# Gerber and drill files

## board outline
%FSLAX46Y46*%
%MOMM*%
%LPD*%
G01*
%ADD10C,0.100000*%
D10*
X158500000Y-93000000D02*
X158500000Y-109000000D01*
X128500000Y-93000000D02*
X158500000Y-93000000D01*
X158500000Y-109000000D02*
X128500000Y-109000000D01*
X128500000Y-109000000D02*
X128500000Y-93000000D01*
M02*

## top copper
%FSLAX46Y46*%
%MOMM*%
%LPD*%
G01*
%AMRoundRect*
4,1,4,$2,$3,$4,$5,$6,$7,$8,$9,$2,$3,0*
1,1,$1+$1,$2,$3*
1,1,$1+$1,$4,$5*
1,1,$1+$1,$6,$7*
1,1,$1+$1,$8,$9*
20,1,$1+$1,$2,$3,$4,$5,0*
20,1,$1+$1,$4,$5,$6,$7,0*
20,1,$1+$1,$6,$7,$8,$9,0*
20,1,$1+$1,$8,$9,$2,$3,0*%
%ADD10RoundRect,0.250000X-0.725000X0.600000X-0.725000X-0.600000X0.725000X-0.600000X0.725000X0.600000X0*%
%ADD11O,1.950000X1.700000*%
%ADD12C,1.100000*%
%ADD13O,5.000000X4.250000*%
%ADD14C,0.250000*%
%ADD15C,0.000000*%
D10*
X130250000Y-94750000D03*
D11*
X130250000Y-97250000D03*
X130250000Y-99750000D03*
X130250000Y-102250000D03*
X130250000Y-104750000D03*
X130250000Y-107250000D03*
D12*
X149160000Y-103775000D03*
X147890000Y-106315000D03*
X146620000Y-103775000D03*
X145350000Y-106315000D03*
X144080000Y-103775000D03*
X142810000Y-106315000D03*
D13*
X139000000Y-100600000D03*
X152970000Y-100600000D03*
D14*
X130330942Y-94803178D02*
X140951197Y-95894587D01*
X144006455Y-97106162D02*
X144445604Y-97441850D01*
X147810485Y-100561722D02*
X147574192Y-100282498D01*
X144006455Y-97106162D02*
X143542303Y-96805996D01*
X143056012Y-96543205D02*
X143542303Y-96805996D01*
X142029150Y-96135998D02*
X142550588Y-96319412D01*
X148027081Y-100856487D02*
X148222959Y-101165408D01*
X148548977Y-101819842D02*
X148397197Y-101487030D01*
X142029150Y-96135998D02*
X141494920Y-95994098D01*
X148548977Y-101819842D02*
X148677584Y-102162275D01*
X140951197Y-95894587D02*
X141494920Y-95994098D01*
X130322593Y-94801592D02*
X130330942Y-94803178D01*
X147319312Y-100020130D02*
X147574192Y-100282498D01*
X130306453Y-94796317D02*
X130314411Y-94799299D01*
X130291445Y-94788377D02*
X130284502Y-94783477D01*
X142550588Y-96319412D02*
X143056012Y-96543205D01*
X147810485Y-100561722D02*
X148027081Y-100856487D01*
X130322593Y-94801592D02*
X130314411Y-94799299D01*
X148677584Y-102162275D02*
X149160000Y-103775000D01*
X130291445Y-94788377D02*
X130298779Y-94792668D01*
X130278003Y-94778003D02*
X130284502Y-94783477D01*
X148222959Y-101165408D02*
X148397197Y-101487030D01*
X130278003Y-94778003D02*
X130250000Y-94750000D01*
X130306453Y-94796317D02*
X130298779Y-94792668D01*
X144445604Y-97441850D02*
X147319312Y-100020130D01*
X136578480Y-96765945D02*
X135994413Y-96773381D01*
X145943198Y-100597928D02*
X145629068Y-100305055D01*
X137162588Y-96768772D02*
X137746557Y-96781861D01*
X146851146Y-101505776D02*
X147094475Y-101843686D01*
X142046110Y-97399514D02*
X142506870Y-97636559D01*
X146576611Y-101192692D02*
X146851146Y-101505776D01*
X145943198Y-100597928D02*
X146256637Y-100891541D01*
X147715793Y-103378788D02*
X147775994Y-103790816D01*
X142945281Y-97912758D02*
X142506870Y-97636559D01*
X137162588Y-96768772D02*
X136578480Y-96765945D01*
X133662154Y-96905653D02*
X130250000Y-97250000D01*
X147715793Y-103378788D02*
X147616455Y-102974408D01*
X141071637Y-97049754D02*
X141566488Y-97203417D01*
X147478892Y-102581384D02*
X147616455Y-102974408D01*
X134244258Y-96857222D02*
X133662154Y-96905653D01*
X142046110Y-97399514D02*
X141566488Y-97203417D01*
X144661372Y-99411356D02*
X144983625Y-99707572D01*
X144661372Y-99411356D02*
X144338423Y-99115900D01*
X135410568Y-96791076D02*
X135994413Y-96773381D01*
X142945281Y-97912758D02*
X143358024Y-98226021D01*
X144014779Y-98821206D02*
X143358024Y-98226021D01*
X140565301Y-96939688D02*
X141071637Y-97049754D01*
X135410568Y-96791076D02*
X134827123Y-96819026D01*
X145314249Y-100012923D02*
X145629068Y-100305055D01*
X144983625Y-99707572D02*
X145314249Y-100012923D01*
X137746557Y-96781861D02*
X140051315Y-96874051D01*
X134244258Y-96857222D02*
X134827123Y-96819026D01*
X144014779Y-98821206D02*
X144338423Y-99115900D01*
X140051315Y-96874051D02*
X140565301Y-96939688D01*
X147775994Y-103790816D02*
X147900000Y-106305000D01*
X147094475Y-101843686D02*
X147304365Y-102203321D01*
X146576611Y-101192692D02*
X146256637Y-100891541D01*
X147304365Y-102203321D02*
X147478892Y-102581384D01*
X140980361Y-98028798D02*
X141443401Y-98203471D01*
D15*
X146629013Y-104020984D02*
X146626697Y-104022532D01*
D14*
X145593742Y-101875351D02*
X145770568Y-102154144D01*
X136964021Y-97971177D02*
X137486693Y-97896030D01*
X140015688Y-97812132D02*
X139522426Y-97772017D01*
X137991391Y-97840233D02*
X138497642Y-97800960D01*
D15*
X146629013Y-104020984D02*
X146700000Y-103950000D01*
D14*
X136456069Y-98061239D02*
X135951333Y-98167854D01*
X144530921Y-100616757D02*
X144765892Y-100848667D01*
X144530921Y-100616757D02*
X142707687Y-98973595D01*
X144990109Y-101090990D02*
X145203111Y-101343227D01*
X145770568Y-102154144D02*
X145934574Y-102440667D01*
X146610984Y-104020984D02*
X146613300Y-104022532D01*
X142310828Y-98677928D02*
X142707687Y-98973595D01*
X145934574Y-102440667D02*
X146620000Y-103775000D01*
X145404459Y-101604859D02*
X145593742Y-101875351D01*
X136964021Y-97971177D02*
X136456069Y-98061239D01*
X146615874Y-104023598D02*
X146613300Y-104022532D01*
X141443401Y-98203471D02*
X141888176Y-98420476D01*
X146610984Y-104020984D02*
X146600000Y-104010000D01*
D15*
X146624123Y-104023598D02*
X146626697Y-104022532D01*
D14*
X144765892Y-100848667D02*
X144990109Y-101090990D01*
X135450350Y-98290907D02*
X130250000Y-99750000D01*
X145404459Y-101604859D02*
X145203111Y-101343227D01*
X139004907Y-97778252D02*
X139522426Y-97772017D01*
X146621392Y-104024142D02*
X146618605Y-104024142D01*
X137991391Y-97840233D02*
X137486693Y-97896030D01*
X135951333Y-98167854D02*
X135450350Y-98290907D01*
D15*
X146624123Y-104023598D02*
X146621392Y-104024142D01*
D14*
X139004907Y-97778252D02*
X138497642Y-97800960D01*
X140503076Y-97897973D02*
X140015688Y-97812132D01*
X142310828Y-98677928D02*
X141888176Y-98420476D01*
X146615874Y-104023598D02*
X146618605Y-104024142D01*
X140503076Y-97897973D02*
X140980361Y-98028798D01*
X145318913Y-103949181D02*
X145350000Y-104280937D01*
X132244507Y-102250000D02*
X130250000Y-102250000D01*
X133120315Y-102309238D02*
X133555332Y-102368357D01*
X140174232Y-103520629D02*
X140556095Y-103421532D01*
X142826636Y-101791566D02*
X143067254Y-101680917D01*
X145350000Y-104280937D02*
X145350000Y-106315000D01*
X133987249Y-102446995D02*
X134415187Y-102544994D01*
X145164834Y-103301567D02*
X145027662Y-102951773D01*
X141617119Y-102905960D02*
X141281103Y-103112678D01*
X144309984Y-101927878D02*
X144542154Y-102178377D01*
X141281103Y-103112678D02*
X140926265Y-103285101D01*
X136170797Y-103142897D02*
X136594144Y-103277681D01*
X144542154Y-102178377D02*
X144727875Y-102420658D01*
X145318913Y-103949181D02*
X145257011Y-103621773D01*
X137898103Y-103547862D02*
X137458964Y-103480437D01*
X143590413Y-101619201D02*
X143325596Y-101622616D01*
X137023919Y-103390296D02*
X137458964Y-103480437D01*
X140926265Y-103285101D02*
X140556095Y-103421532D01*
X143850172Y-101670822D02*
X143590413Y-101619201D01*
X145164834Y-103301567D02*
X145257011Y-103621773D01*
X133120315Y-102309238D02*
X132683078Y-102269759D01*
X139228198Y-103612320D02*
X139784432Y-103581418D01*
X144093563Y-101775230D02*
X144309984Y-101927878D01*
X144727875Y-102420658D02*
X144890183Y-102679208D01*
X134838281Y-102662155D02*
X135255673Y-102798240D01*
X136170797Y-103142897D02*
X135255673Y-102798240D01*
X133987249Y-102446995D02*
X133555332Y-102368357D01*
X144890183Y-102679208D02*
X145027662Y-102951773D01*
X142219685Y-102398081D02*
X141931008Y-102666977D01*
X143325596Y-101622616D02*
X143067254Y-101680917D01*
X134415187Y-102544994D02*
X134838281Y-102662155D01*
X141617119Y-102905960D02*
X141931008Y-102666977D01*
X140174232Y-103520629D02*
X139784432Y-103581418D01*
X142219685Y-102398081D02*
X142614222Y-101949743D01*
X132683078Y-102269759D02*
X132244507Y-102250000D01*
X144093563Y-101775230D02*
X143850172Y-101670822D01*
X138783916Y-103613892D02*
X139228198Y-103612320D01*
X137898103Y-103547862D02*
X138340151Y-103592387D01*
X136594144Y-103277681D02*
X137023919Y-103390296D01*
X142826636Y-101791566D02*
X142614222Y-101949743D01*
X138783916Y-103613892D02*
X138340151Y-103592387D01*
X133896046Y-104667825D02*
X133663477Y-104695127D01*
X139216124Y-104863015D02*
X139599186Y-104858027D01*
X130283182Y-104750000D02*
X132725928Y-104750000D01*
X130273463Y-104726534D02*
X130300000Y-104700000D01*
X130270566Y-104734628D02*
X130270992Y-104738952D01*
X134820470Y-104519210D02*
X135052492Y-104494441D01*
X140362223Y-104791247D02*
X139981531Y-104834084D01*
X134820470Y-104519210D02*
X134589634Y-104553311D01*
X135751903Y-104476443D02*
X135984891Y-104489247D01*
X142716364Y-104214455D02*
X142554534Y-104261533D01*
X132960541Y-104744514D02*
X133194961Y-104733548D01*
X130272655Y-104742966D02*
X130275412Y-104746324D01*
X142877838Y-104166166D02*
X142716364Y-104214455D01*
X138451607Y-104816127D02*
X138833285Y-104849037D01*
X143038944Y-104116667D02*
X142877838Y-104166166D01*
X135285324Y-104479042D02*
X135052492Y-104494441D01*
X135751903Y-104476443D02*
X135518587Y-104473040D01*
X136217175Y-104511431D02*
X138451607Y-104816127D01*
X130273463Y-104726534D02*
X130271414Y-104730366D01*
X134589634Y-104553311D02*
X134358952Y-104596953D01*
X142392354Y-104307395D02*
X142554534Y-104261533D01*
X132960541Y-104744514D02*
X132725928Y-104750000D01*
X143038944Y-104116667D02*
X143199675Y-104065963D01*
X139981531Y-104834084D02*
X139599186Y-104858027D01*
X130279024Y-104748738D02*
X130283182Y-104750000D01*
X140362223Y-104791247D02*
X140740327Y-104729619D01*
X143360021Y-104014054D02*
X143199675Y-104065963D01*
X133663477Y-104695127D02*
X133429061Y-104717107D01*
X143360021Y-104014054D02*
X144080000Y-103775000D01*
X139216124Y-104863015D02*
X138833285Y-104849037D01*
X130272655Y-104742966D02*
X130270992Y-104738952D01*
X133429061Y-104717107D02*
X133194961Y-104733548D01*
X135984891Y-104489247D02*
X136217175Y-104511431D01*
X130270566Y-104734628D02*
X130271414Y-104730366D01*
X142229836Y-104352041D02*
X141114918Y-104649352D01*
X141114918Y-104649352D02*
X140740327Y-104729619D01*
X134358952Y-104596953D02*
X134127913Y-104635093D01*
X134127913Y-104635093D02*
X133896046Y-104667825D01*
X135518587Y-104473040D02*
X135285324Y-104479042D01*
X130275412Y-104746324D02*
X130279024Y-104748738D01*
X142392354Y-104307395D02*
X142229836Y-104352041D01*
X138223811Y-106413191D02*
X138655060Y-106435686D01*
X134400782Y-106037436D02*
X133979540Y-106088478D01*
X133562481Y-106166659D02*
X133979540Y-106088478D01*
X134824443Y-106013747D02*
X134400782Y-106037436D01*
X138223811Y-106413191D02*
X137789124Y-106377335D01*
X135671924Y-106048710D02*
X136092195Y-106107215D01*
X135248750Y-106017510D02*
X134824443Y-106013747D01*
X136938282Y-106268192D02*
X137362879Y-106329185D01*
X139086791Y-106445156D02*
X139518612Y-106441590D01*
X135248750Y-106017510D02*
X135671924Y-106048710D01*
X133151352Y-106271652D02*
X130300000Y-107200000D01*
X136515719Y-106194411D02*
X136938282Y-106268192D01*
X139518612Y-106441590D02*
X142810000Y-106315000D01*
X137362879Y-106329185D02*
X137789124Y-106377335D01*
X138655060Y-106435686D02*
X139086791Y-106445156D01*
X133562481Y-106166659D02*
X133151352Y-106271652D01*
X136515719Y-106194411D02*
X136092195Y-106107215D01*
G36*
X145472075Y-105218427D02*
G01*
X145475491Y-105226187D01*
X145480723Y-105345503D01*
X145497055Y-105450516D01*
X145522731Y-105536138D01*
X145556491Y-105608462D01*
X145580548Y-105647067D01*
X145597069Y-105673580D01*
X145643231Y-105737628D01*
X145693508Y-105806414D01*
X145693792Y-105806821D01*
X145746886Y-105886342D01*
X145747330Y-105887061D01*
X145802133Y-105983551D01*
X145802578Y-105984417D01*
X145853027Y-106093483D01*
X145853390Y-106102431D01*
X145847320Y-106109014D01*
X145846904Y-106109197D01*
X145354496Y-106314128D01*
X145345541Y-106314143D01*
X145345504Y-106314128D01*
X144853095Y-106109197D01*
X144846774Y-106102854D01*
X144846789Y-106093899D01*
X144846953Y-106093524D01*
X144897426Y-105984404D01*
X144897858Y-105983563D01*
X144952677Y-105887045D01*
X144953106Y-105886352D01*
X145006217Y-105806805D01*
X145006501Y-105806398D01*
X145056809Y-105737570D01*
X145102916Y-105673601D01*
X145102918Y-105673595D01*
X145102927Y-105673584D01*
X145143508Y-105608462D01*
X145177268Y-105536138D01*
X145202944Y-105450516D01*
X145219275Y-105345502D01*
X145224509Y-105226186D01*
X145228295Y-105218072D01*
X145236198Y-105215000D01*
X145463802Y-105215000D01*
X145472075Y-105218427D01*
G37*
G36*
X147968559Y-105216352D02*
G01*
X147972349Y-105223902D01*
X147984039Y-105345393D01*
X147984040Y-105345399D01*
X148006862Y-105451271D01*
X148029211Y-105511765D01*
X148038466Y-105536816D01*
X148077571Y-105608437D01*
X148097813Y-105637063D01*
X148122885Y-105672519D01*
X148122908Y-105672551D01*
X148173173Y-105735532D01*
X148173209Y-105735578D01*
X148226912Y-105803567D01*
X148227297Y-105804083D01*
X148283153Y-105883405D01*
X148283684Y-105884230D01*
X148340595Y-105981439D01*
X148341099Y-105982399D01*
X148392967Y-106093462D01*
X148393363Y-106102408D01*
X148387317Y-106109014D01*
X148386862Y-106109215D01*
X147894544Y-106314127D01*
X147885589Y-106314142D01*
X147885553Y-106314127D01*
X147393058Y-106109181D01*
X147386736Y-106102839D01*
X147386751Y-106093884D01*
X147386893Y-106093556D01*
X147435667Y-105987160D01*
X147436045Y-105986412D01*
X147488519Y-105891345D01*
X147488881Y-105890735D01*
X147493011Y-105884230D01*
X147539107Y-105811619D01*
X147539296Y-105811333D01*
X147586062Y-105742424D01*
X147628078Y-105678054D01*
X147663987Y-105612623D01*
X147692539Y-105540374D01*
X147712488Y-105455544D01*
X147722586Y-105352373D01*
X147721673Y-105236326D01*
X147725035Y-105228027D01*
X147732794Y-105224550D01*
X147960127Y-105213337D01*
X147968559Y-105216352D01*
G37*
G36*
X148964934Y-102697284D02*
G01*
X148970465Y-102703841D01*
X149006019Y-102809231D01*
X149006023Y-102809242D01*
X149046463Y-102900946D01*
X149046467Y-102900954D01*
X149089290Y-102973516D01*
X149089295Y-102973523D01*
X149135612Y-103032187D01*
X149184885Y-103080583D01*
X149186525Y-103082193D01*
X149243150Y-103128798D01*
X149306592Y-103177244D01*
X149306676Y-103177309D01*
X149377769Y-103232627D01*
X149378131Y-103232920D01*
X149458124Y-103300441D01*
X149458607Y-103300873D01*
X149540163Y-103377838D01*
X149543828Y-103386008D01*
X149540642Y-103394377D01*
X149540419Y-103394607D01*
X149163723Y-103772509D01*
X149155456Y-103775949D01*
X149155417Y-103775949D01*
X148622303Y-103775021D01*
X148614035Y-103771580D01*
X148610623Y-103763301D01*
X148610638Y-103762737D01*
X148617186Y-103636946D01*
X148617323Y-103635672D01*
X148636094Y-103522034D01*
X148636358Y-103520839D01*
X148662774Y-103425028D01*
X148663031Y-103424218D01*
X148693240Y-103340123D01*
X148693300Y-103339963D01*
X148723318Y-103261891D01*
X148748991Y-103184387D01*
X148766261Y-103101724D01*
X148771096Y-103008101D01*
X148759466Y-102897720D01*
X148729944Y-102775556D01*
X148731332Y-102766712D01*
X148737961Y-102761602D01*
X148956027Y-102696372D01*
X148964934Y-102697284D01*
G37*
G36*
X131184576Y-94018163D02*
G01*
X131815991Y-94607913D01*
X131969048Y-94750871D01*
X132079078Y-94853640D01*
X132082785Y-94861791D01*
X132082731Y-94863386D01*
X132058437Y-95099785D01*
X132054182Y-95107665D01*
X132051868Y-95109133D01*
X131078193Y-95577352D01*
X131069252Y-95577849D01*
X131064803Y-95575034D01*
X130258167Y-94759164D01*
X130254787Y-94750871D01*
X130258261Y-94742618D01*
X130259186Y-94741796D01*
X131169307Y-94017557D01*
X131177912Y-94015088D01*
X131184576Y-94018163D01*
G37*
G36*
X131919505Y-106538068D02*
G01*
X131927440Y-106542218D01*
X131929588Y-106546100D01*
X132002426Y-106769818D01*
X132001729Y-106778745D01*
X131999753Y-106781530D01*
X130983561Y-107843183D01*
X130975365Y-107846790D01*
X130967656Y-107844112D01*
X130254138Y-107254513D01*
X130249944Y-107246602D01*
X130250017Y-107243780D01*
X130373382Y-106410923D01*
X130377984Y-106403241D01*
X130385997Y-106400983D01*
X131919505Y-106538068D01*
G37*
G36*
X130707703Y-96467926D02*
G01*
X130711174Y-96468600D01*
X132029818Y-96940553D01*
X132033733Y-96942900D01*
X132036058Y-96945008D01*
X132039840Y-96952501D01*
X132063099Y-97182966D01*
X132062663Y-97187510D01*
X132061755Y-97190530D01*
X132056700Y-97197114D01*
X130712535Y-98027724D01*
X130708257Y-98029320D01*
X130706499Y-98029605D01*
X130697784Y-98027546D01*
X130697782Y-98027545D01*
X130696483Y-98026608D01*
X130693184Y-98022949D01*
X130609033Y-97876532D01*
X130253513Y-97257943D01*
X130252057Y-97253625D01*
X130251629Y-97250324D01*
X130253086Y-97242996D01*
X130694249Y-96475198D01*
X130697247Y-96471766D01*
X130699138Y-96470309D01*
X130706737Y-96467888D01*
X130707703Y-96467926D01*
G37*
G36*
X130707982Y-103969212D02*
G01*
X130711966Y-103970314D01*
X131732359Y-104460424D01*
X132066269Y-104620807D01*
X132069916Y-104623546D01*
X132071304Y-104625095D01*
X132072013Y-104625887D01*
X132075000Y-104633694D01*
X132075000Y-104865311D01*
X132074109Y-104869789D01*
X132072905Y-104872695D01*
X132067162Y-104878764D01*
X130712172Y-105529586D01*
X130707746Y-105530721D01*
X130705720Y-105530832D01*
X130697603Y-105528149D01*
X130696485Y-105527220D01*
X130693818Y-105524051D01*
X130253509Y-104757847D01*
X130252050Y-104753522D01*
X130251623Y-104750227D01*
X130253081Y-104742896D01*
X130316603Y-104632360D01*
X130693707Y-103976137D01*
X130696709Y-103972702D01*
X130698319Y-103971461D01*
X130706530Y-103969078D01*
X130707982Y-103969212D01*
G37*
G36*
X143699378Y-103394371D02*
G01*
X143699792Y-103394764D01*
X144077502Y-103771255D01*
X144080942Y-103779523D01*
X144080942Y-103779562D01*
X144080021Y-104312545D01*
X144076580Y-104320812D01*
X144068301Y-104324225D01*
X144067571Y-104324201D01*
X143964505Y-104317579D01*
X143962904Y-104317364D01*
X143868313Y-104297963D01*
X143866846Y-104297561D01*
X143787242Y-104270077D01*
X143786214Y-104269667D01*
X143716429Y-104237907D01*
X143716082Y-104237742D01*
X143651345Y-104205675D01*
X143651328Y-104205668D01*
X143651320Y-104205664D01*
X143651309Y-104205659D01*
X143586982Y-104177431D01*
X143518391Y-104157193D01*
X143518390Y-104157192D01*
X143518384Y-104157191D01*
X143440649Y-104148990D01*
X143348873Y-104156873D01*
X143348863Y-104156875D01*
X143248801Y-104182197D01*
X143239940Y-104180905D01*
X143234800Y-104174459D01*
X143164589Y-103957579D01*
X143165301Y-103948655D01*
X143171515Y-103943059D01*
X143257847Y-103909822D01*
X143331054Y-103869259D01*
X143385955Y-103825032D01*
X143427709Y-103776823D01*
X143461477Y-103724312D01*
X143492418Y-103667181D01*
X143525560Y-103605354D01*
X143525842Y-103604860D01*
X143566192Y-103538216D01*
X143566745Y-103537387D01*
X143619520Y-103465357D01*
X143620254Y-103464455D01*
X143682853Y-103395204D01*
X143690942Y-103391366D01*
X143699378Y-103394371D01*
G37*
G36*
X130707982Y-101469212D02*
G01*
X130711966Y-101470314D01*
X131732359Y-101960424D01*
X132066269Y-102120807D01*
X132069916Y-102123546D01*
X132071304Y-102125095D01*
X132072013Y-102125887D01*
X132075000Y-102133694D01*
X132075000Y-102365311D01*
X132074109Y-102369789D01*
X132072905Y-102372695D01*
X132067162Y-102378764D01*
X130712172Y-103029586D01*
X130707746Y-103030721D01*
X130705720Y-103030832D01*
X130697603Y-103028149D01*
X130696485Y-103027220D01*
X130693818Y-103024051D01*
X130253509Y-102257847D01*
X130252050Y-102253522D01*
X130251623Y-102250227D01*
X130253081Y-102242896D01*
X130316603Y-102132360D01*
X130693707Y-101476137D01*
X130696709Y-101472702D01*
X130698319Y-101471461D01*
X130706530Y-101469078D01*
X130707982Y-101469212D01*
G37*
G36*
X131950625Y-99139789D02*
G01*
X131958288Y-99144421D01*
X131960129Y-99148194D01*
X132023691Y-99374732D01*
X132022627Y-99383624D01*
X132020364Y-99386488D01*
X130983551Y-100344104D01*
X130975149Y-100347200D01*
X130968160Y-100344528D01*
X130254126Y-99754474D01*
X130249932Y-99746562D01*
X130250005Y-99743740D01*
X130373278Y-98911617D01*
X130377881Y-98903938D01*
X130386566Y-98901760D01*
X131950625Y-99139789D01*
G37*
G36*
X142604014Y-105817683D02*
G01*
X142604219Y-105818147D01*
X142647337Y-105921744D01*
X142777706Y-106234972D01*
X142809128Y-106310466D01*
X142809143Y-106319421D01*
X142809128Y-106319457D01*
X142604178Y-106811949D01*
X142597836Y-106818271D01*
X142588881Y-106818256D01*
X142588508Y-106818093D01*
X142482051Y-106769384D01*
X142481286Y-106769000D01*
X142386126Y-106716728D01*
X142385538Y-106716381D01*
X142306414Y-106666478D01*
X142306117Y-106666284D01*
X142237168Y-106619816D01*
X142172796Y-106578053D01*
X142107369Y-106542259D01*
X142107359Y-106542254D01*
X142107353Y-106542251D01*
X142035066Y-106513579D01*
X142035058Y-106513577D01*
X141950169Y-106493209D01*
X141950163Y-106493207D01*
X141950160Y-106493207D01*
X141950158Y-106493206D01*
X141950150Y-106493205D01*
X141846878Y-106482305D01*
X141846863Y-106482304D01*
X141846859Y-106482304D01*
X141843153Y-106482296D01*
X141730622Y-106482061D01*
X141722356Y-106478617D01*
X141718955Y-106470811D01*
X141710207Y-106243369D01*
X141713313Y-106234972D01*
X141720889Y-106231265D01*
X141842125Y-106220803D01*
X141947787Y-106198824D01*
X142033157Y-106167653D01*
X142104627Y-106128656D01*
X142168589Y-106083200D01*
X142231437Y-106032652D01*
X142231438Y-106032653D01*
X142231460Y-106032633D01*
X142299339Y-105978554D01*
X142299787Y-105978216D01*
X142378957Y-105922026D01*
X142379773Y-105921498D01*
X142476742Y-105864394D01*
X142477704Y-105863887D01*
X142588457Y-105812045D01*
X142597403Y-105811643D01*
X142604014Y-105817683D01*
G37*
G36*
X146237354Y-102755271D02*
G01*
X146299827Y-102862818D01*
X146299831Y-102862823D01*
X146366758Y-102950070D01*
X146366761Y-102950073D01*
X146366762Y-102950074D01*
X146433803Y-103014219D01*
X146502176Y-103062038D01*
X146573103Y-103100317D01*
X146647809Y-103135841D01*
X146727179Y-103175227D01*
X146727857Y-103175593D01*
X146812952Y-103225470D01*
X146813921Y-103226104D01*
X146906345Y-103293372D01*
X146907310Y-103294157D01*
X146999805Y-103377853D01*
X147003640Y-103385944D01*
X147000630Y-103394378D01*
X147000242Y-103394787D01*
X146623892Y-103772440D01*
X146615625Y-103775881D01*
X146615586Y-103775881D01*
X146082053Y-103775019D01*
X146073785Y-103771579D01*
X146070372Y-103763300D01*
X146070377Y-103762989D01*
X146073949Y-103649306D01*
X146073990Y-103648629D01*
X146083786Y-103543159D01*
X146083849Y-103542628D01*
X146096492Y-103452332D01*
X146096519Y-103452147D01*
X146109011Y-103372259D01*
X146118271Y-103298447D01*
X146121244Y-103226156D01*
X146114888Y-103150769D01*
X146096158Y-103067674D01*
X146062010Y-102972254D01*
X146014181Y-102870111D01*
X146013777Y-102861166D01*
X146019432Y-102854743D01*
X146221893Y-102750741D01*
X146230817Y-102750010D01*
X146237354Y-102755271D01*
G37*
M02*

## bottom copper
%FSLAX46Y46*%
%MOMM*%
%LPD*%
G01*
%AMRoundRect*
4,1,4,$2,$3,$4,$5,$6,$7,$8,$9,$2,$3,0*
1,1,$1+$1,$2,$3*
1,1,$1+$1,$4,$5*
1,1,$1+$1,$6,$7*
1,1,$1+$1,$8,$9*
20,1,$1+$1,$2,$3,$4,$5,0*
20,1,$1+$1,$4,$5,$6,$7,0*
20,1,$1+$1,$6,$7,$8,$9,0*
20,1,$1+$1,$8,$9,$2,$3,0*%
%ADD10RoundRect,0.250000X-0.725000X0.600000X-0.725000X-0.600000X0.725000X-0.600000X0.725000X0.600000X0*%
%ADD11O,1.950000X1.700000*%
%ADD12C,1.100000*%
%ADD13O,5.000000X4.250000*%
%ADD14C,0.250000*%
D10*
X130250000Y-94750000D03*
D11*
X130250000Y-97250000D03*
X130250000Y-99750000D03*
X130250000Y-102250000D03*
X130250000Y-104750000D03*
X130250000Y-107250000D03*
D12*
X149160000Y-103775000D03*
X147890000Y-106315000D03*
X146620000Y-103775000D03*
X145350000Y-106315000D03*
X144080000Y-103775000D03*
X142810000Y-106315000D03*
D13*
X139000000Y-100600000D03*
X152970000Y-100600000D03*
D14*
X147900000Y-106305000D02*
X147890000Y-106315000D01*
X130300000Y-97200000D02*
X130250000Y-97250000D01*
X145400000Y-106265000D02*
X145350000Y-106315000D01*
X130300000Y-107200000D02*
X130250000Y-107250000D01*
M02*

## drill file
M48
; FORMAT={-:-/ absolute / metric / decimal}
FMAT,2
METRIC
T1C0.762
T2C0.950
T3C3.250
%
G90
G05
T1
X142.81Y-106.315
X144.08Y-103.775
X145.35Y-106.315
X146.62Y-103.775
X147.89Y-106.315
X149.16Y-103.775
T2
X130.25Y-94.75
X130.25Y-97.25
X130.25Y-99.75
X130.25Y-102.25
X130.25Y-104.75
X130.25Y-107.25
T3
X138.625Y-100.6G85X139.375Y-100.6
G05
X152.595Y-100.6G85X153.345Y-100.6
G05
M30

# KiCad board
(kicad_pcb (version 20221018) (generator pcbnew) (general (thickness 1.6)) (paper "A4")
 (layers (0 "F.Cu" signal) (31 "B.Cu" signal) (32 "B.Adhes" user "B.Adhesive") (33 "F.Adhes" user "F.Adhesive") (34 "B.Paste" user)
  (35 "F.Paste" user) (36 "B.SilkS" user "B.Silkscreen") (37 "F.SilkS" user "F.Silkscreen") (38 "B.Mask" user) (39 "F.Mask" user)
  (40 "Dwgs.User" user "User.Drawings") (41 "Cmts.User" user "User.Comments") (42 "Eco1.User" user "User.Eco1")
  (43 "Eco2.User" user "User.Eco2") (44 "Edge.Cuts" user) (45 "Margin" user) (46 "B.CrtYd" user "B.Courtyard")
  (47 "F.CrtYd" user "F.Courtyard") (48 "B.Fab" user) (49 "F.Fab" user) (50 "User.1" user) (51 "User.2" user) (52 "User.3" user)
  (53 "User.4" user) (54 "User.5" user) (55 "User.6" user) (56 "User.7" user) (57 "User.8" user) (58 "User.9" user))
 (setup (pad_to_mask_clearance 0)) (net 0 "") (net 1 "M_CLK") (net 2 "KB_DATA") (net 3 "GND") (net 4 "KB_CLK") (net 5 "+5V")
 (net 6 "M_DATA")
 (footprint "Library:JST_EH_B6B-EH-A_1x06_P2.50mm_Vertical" (layer "F.Cu") (at 130.25 94.75 -90)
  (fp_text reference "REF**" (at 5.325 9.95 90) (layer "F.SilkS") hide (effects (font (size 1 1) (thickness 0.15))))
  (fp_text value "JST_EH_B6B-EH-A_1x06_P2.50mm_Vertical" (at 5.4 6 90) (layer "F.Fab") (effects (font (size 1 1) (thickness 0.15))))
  (pad "1" thru_hole roundrect (at 0 0 270) (size 1.7 1.95) (drill 0.95) (layers "*.Cu" "*.Mask") (roundrect_rratio 0.1470588235)
   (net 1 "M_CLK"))
  (pad "2" thru_hole oval (at 2.5 0 270) (size 1.7 1.95) (drill 0.95) (layers "*.Cu" "*.Mask") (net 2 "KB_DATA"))
  (pad "3" thru_hole oval (at 5 0 270) (size 1.7 1.95) (drill 0.95) (layers "*.Cu" "*.Mask") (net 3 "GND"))
  (pad "4" thru_hole oval (at 7.5 0 270) (size 1.7 1.95) (drill 0.95) (layers "*.Cu" "*.Mask") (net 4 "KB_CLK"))
  (pad "5" thru_hole oval (at 10 0 270) (size 1.7 1.95) (drill 0.95) (layers "*.Cu" "*.Mask") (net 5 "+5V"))
  (pad "6" thru_hole oval (at 12.5 0 270) (size 1.7 1.95) (drill 0.95) (layers "*.Cu" "*.Mask") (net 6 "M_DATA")))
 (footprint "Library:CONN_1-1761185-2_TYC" (layer "F.Cu") (at 142.81 106.315)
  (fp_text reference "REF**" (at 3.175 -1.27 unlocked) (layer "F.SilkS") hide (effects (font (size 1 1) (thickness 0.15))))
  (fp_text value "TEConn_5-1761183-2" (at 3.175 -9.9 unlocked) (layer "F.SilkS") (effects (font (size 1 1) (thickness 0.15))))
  (pad "1" thru_hole circle (at 6.35 -2.54) (size 1.1 1.1) (drill 0.762) (layers "*.Cu" "*.Mask") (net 1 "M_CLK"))
  (pad "2" thru_hole circle (at 5.08 0) (size 1.1 1.1) (drill 0.762) (layers "*.Cu" "*.Mask") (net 2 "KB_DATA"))
  (pad "3" thru_hole circle (at 3.81 -2.54) (size 1.1 1.1) (drill 0.762) (layers "*.Cu" "*.Mask") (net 3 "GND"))
  (pad "4" thru_hole circle (at 2.54 0) (size 1.1 1.1) (drill 0.762) (layers "*.Cu" "*.Mask") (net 4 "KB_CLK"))
  (pad "5" thru_hole circle (at 1.27 -2.54) (size 1.1 1.1) (drill 0.762) (layers "*.Cu" "*.Mask") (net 5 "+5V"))
  (pad "6" thru_hole circle (at 0 0) (size 1.1 1.1) (drill 0.762) (layers "*.Cu" "*.Mask") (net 6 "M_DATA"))
  (pad "13" thru_hole oval (at -3.81 -5.715) (size 5 4.25) (drill oval 4 3.25) (layers "*.Cu" "*.Mask"))
  (pad "14" thru_hole oval (at 10.16 -5.715) (size 5 4.25) (drill oval 4 3.25) (layers "*.Cu" "*.Mask")))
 (gr_line (start 158.5 93) (end 158.5 109) (stroke (width 0.1) (type default)) (layer "Edge.Cuts"))
 (gr_line (start 128.5 93) (end 158.5 93) (stroke (width 0.1) (type default)) (layer "Edge.Cuts"))
 (gr_line (start 158.5 109) (end 128.5 109) (stroke (width 0.1) (type default)) (layer "Edge.Cuts"))
 (gr_line (start 128.5 109) (end 128.5 93) (stroke (width 0.1) (type default)) (layer "Edge.Cuts"))
 (segment (start 130.330942 94.803178) (end 140.951197 95.894587) (width 0.25) (layer "F.Cu") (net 1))
 (segment (start 144.006455 97.106162) (end 144.445604 97.44185) (width 0.25) (layer "F.Cu") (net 1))
 (segment (start 147.810485 100.561722) (end 147.574192 100.282498) (width 0.25) (layer "F.Cu") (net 1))
 (segment (start 144.006455 97.106162) (end 143.542303 96.805996) (width 0.25) (layer "F.Cu") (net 1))
 (segment (start 143.056012 96.543205) (end 143.542303 96.805996) (width 0.25) (layer "F.Cu") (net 1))
 (segment (start 142.02915 96.135998) (end 142.550588 96.319412) (width 0.25) (layer "F.Cu") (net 1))
 (segment (start 148.027081 100.856487) (end 148.222959 101.165408) (width 0.25) (layer "F.Cu") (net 1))
 (segment (start 148.548977 101.819842) (end 148.397197 101.48703) (width 0.25) (layer "F.Cu") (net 1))
 (segment (start 142.02915 96.135998) (end 141.49492 95.994098) (width 0.25) (layer "F.Cu") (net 1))
 (segment (start 148.548977 101.819842) (end 148.677584 102.162275) (width 0.25) (layer "F.Cu") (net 1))
 (segment (start 140.951197 95.894587) (end 141.49492 95.994098) (width 0.25) (layer "F.Cu") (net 1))
 (segment (start 130.322593 94.801592) (end 130.330942 94.803178) (width 0.25) (layer "F.Cu") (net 1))
 (segment (start 147.319312 100.02013) (end 147.574192 100.282498) (width 0.25) (layer "F.Cu") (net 1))
 (segment (start 130.306453 94.796317) (end 130.314411 94.799299) (width 0.25) (layer "F.Cu") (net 1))
 (segment (start 130.291445 94.788377) (end 130.284502 94.783477) (width 0.25) (layer "F.Cu") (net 1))
 (segment (start 142.550588 96.319412) (end 143.056012 96.543205) (width 0.25) (layer "F.Cu") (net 1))
 (segment (start 147.810485 100.561722) (end 148.027081 100.856487) (width 0.25) (layer "F.Cu") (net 1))
 (segment (start 130.322593 94.801592) (end 130.314411 94.799299) (width 0.25) (layer "F.Cu") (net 1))
 (segment (start 148.677584 102.162275) (end 149.16 103.775) (width 0.25) (layer "F.Cu") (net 1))
 (segment (start 130.291445 94.788377) (end 130.298779 94.792668) (width 0.25) (layer "F.Cu") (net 1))
 (segment (start 130.278003 94.778003) (end 130.284502 94.783477) (width 0.25) (layer "F.Cu") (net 1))
 (segment (start 148.222959 101.165408) (end 148.397197 101.48703) (width 0.25) (layer "F.Cu") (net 1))
 (segment (start 130.278003 94.778003) (end 130.25 94.75) (width 0.25) (layer "F.Cu") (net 1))
 (segment (start 130.306453 94.796317) (end 130.298779 94.792668) (width 0.25) (layer "F.Cu") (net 1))
 (segment (start 144.445604 97.44185) (end 147.319312 100.02013) (width 0.25) (layer "F.Cu") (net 1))
 (segment (start 136.57848 96.765945) (end 135.994413 96.773381) (width 0.25) (layer "F.Cu") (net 2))
 (segment (start 145.943198 100.597928) (end 145.629068 100.305055) (width 0.25) (layer "F.Cu") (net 2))
 (segment (start 137.162588 96.768772) (end 137.746557 96.781861) (width 0.25) (layer "F.Cu") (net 2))
 (segment (start 146.851146 101.505776) (end 147.094475 101.843686) (width 0.25) (layer "F.Cu") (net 2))
 (segment (start 142.04611 97.399514) (end 142.50687 97.636559) (width 0.25) (layer "F.Cu") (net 2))
 (segment (start 146.576611 101.192692) (end 146.851146 101.505776) (width 0.25) (layer "F.Cu") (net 2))
 (segment (start 145.943198 100.597928) (end 146.256637 100.891541) (width 0.25) (layer "F.Cu") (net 2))
 (segment (start 147.715793 103.378788) (end 147.775994 103.790816) (width 0.25) (layer "F.Cu") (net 2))
 (segment (start 142.945281 97.912758) (end 142.50687 97.636559) (width 0.25) (layer "F.Cu") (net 2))
 (segment (start 137.162588 96.768772) (end 136.57848 96.765945) (width 0.25) (layer "F.Cu") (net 2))
 (segment (start 133.662154 96.905653) (end 130.25 97.25) (width 0.25) (layer "F.Cu") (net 2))
 (segment (start 147.715793 103.378788) (end 147.616455 102.974408) (width 0.25) (layer "F.Cu") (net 2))
 (segment (start 141.071637 97.049754) (end 141.566488 97.203417) (width 0.25) (layer "F.Cu") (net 2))
 (segment (start 147.478892 102.581384) (end 147.616455 102.974408) (width 0.25) (layer "F.Cu") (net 2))
 (segment (start 134.244258 96.857222) (end 133.662154 96.905653) (width 0.25) (layer "F.Cu") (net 2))
 (segment (start 142.04611 97.399514) (end 141.566488 97.203417) (width 0.25) (layer "F.Cu") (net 2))
 (segment (start 144.661372 99.411356) (end 144.983625 99.707572) (width 0.25) (layer "F.Cu") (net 2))
 (segment (start 144.661372 99.411356) (end 144.338423 99.1159) (width 0.25) (layer "F.Cu") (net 2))
 (segment (start 135.410568 96.791076) (end 135.994413 96.773381) (width 0.25) (layer "F.Cu") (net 2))
 (segment (start 142.945281 97.912758) (end 143.358024 98.226021) (width 0.25) (layer "F.Cu") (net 2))
 (segment (start 144.014779 98.821206) (end 143.358024 98.226021) (width 0.25) (layer "F.Cu") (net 2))
 (segment (start 140.565301 96.939688) (end 141.071637 97.049754) (width 0.25) (layer "F.Cu") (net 2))
 (segment (start 135.410568 96.791076) (end 134.827123 96.819026) (width 0.25) (layer "F.Cu") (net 2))
 (segment (start 145.314249 100.012923) (end 145.629068 100.305055) (width 0.25) (layer "F.Cu") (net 2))
 (segment (start 144.983625 99.707572) (end 145.314249 100.012923) (width 0.25) (layer "F.Cu") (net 2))
 (segment (start 137.746557 96.781861) (end 140.051315 96.874051) (width 0.25) (layer "F.Cu") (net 2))
 (segment (start 134.244258 96.857222) (end 134.827123 96.819026) (width 0.25) (layer "F.Cu") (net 2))
 (segment (start 144.014779 98.821206) (end 144.338423 99.1159) (width 0.25) (layer "F.Cu") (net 2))
 (segment (start 140.051315 96.874051) (end 140.565301 96.939688) (width 0.25) (layer "F.Cu") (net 2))
 (segment (start 147.775994 103.790816) (end 147.9 106.305) (width 0.25) (layer "F.Cu") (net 2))
 (segment (start 147.094475 101.843686) (end 147.304365 102.203321) (width 0.25) (layer "F.Cu") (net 2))
 (segment (start 146.576611 101.192692) (end 146.256637 100.891541) (width 0.25) (layer "F.Cu") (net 2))
 (segment (start 147.304365 102.203321) (end 147.478892 102.581384) (width 0.25) (layer "F.Cu") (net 2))
 (segment (start 147.9 106.305) (end 147.89 106.315) (width 0.25) (layer "B.Cu") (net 2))
 (segment (start 130.3 97.2) (end 130.25 97.25) (width 0.25) (layer "B.Cu") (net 2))
 (segment (start 140.980361 98.028798) (end 141.443401 98.203471) (width 0.25) (layer "F.Cu") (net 3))
 (segment (start 146.629013 104.020984) (end 146.626697 104.022532) (width 0) (layer "F.Cu") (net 3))
 (segment (start 145.593742 101.875351) (end 145.770568 102.154144) (width 0.25) (layer "F.Cu") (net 3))
 (segment (start 136.964021 97.971177) (end 137.486693 97.89603) (width 0.25) (layer "F.Cu") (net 3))
 (segment (start 140.015688 97.812132) (end 139.522426 97.772017) (width 0.25) (layer "F.Cu") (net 3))
 (segment (start 137.991391 97.840233) (end 138.497642 97.80096) (width 0.25) (layer "F.Cu") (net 3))
 (segment (start 146.629013 104.020984) (end 146.7 103.95) (width 0) (layer "F.Cu") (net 3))
 (segment (start 136.456069 98.061239) (end 135.951333 98.167854) (width 0.25) (layer "F.Cu") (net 3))
 (segment (start 144.530921 100.616757) (end 144.765892 100.848667) (width 0.25) (layer "F.Cu") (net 3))
 (segment (start 144.530921 100.616757) (end 142.707687 98.973595) (width 0.25) (layer "F.Cu") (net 3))
 (segment (start 144.990109 101.09099) (end 145.203111 101.343227) (width 0.25) (layer "F.Cu") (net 3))
 (segment (start 145.770568 102.154144) (end 145.934574 102.440667) (width 0.25) (layer "F.Cu") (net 3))
 (segment (start 146.610984 104.020984) (end 146.6133 104.022532) (width 0.25) (layer "F.Cu") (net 3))
 (segment (start 142.310828 98.677928) (end 142.707687 98.973595) (width 0.25) (layer "F.Cu") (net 3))
 (segment (start 145.934574 102.440667) (end 146.62 103.775) (width 0.25) (layer "F.Cu") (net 3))
 (segment (start 145.404459 101.604859) (end 145.593742 101.875351) (width 0.25) (layer "F.Cu") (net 3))
 (segment (start 136.964021 97.971177) (end 136.456069 98.061239) (width 0.25) (layer "F.Cu") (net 3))
 (segment (start 146.615874 104.023598) (end 146.6133 104.022532) (width 0.25) (layer "F.Cu") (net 3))
 (segment (start 141.443401 98.203471) (end 141.888176 98.420476) (width 0.25) (layer "F.Cu") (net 3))
 (segment (start 146.610984 104.020984) (end 146.6 104.01) (width 0.25) (layer "F.Cu") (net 3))
 (segment (start 146.624123 104.023598) (end 146.626697 104.022532) (width 0) (layer "F.Cu") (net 3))
 (segment (start 144.765892 100.848667) (end 144.990109 101.09099) (width 0.25) (layer "F.Cu") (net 3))
 (segment (start 135.45035 98.290907) (end 130.25 99.75) (width 0.25) (layer "F.Cu") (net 3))
 (segment (start 145.404459 101.604859) (end 145.203111 101.343227) (width 0.25) (layer "F.Cu") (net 3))
 (segment (start 139.004907 97.778252) (end 139.522426 97.772017) (width 0.25) (layer "F.Cu") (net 3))
 (segment (start 146.621392 104.024142) (end 146.618605 104.024142) (width 0.25) (layer "F.Cu") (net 3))
 (segment (start 137.991391 97.840233) (end 137.486693 97.89603) (width 0.25) (layer "F.Cu") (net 3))
 (segment (start 135.951333 98.167854) (end 135.45035 98.290907) (width 0.25) (layer "F.Cu") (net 3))
 (segment (start 146.624123 104.023598) (end 146.621392 104.024142) (width 0) (layer "F.Cu") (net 3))
 (segment (start 139.004907 97.778252) (end 138.497642 97.80096) (width 0.25) (layer "F.Cu") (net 3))
 (segment (start 140.503076 97.897973) (end 140.015688 97.812132) (width 0.25) (layer "F.Cu") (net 3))
 (segment (start 142.310828 98.677928) (end 141.888176 98.420476) (width 0.25) (layer "F.Cu") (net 3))
 (segment (start 146.615874 104.023598) (end 146.618605 104.024142) (width 0.25) (layer "F.Cu") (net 3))
 (segment (start 140.503076 97.897973) (end 140.980361 98.028798) (width 0.25) (layer "F.Cu") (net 3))
 (segment (start 145.318913 103.949181) (end 145.35 104.280937) (width 0.25) (layer "F.Cu") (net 4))
 (segment (start 132.244507 102.25) (end 130.25 102.25) (width 0.25) (layer "F.Cu") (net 4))
 (segment (start 133.120315 102.309238) (end 133.555332 102.368357) (width 0.25) (layer "F.Cu") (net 4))
 (segment (start 140.174232 103.520629) (end 140.556095 103.421532) (width 0.25) (layer "F.Cu") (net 4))
 (segment (start 142.826636 101.791566) (end 143.067254 101.680917) (width 0.25) (layer "F.Cu") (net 4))
 (segment (start 145.35 104.280937) (end 145.35 106.315) (width 0.25) (layer "F.Cu") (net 4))
 (segment (start 133.987249 102.446995) (end 134.415187 102.544994) (width 0.25) (layer "F.Cu") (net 4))
 (segment (start 145.164834 103.301567) (end 145.027662 102.951773) (width 0.25) (layer "F.Cu") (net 4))
 (segment (start 141.617119 102.90596) (end 141.281103 103.112678) (width 0.25) (layer "F.Cu") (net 4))
 (segment (start 144.309984 101.927878) (end 144.542154 102.178377) (width 0.25) (layer "F.Cu") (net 4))
 (segment (start 141.281103 103.112678) (end 140.926265 103.285101) (width 0.25) (layer "F.Cu") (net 4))
 (segment (start 136.170797 103.142897) (end 136.594144 103.277681) (width 0.25) (layer "F.Cu") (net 4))
 (segment (start 144.542154 102.178377) (end 144.727875 102.420658) (width 0.25) (layer "F.Cu") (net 4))
 (segment (start 145.318913 103.949181) (end 145.257011 103.621773) (width 0.25) (layer "F.Cu") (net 4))
 (segment (start 137.898103 103.547862) (end 137.458964 103.480437) (width 0.25) (layer "F.Cu") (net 4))
 (segment (start 143.590413 101.619201) (end 143.325596 101.622616) (width 0.25) (layer "F.Cu") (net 4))
 (segment (start 137.023919 103.390296) (end 137.458964 103.480437) (width 0.25) (layer "F.Cu") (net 4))
 (segment (start 140.926265 103.285101) (end 140.556095 103.421532) (width 0.25) (layer "F.Cu") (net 4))
 (segment (start 143.850172 101.670822) (end 143.590413 101.619201) (width 0.25) (layer "F.Cu") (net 4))
 (segment (start 145.164834 103.301567) (end 145.257011 103.621773) (width 0.25) (layer "F.Cu") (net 4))
 (segment (start 133.120315 102.309238) (end 132.683078 102.269759) (width 0.25) (layer "F.Cu") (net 4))
 (segment (start 139.228198 103.61232) (end 139.784432 103.581418) (width 0.25) (layer "F.Cu") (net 4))
 (segment (start 144.093563 101.77523) (end 144.309984 101.927878) (width 0.25) (layer "F.Cu") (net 4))
 (segment (start 144.727875 102.420658) (end 144.890183 102.679208) (width 0.25) (layer "F.Cu") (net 4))
 (segment (start 134.838281 102.662155) (end 135.255673 102.79824) (width 0.25) (layer "F.Cu") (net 4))
 (segment (start 136.170797 103.142897) (end 135.255673 102.79824) (width 0.25) (layer "F.Cu") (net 4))
 (segment (start 133.987249 102.446995) (end 133.555332 102.368357) (width 0.25) (layer "F.Cu") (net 4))
 (segment (start 144.890183 102.679208) (end 145.027662 102.951773) (width 0.25) (layer "F.Cu") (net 4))
 (segment (start 142.219685 102.398081) (end 141.931008 102.666977) (width 0.25) (layer "F.Cu") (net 4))
 (segment (start 143.325596 101.622616) (end 143.067254 101.680917) (width 0.25) (layer "F.Cu") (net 4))
 (segment (start 134.415187 102.544994) (end 134.838281 102.662155) (width 0.25) (layer "F.Cu") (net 4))
 (segment (start 141.617119 102.90596) (end 141.931008 102.666977) (width 0.25) (layer "F.Cu") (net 4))
 (segment (start 140.174232 103.520629) (end 139.784432 103.581418) (width 0.25) (layer "F.Cu") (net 4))
 (segment (start 142.219685 102.398081) (end 142.614222 101.949743) (width 0.25) (layer "F.Cu") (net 4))
 (segment (start 132.683078 102.269759) (end 132.244507 102.25) (width 0.25) (layer "F.Cu") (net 4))
 (segment (start 144.093563 101.77523) (end 143.850172 101.670822) (width 0.25) (layer "F.Cu") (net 4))
 (segment (start 138.783916 103.613892) (end 139.228198 103.61232) (width 0.25) (layer "F.Cu") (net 4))
 (segment (start 137.898103 103.547862) (end 138.340151 103.592387) (width 0.25) (layer "F.Cu") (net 4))
 (segment (start 136.594144 103.277681) (end 137.023919 103.390296) (width 0.25) (layer "F.Cu") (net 4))
 (segment (start 142.826636 101.791566) (end 142.614222 101.949743) (width 0.25) (layer "F.Cu") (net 4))
 (segment (start 138.783916 103.613892) (end 138.340151 103.592387) (width 0.25) (layer "F.Cu") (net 4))
 (segment (start 145.4 106.265) (end 145.35 106.315) (width 0.25) (layer "B.Cu") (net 4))
 (segment (start 133.896046 104.667825) (end 133.663477 104.695127) (width 0.25) (layer "F.Cu") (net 5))
 (segment (start 139.216124 104.863015) (end 139.599186 104.858027) (width 0.25) (layer "F.Cu") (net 5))
 (segment (start 130.283182 104.75) (end 132.725928 104.75) (width 0.25) (layer "F.Cu") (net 5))
 (segment (start 130.273463 104.726534) (end 130.3 104.7) (width 0.25) (layer "F.Cu") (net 5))
 (segment (start 130.270566 104.734628) (end 130.270992 104.738952) (width 0.25) (layer "F.Cu") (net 5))
 (segment (start 134.82047 104.51921) (end 135.052492 104.494441) (width 0.25) (layer "F.Cu") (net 5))
 (segment (start 140.362223 104.791247) (end 139.981531 104.834084) (width 0.25) (layer "F.Cu") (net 5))
 (segment (start 134.82047 104.51921) (end 134.589634 104.553311) (width 0.25) (layer "F.Cu") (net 5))
 (segment (start 135.751903 104.476443) (end 135.984891 104.489247) (width 0.25) (layer "F.Cu") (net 5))
 (segment (start 142.716364 104.214455) (end 142.554534 104.261533) (width 0.25) (layer "F.Cu") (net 5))
 (segment (start 132.960541 104.744514) (end 133.194961 104.733548) (width 0.25) (layer "F.Cu") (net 5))
 (segment (start 130.272655 104.742966) (end 130.275412 104.746324) (width 0.25) (layer "F.Cu") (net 5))
 (segment (start 142.877838 104.166166) (end 142.716364 104.214455) (width 0.25) (layer "F.Cu") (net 5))
 (segment (start 138.451607 104.816127) (end 138.833285 104.849037) (width 0.25) (layer "F.Cu") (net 5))
 (segment (start 143.038944 104.116667) (end 142.877838 104.166166) (width 0.25) (layer "F.Cu") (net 5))
 (segment (start 135.285324 104.479042) (end 135.052492 104.494441) (width 0.25) (layer "F.Cu") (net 5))
 (segment (start 135.751903 104.476443) (end 135.518587 104.47304) (width 0.25) (layer "F.Cu") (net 5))
 (segment (start 136.217175 104.511431) (end 138.451607 104.816127) (width 0.25) (layer "F.Cu") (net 5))
 (segment (start 130.273463 104.726534) (end 130.271414 104.730366) (width 0.25) (layer "F.Cu") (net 5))
 (segment (start 134.589634 104.553311) (end 134.358952 104.596953) (width 0.25) (layer "F.Cu") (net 5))
 (segment (start 142.392354 104.307395) (end 142.554534 104.261533) (width 0.25) (layer "F.Cu") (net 5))
 (segment (start 132.960541 104.744514) (end 132.725928 104.75) (width 0.25) (layer "F.Cu") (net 5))
 (segment (start 143.038944 104.116667) (end 143.199675 104.065963) (width 0.25) (layer "F.Cu") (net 5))
 (segment (start 139.981531 104.834084) (end 139.599186 104.858027) (width 0.25) (layer "F.Cu") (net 5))
 (segment (start 130.279024 104.748738) (end 130.283182 104.75) (width 0.25) (layer "F.Cu") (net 5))
 (segment (start 140.362223 104.791247) (end 140.740327 104.729619) (width 0.25) (layer "F.Cu") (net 5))
 (segment (start 143.360021 104.014054) (end 143.199675 104.065963) (width 0.25) (layer "F.Cu") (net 5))
 (segment (start 133.663477 104.695127) (end 133.429061 104.717107) (width 0.25) (layer "F.Cu") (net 5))
 (segment (start 143.360021 104.014054) (end 144.08 103.775) (width 0.25) (layer "F.Cu") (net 5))
 (segment (start 139.216124 104.863015) (end 138.833285 104.849037) (width 0.25) (layer "F.Cu") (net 5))
 (segment (start 130.272655 104.742966) (end 130.270992 104.738952) (width 0.25) (layer "F.Cu") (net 5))
 (segment (start 133.429061 104.717107) (end 133.194961 104.733548) (width 0.25) (layer "F.Cu") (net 5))
 (segment (start 135.984891 104.489247) (end 136.217175 104.511431) (width 0.25) (layer "F.Cu") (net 5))
 (segment (start 130.270566 104.734628) (end 130.271414 104.730366) (width 0.25) (layer "F.Cu") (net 5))
 (segment (start 142.229836 104.352041) (end 141.114918 104.649352) (width 0.25) (layer "F.Cu") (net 5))
 (segment (start 141.114918 104.649352) (end 140.740327 104.729619) (width 0.25) (layer "F.Cu") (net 5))
 (segment (start 134.358952 104.596953) (end 134.127913 104.635093) (width 0.25) (layer "F.Cu") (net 5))
 (segment (start 134.127913 104.635093) (end 133.896046 104.667825) (width 0.25) (layer "F.Cu") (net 5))
 (segment (start 135.518587 104.47304) (end 135.285324 104.479042) (width 0.25) (layer "F.Cu") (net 5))
 (segment (start 130.275412 104.746324) (end 130.279024 104.748738) (width 0.25) (layer "F.Cu") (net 5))
 (segment (start 142.392354 104.307395) (end 142.229836 104.352041) (width 0.25) (layer "F.Cu") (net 5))
 (segment (start 138.223811 106.413191) (end 138.65506 106.435686) (width 0.25) (layer "F.Cu") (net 6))
 (segment (start 134.400782 106.037436) (end 133.97954 106.088478) (width 0.25) (layer "F.Cu") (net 6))
 (segment (start 133.562481 106.166659) (end 133.97954 106.088478) (width 0.25) (layer "F.Cu") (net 6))
 (segment (start 134.824443 106.013747) (end 134.400782 106.037436) (width 0.25) (layer "F.Cu") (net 6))
 (segment (start 138.223811 106.413191) (end 137.789124 106.377335) (width 0.25) (layer "F.Cu") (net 6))
 (segment (start 135.671924 106.04871) (end 136.092195 106.107215) (width 0.25) (layer "F.Cu") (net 6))
 (segment (start 135.24875 106.01751) (end 134.824443 106.013747) (width 0.25) (layer "F.Cu") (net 6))
 (segment (start 136.938282 106.268192) (end 137.362879 106.329185) (width 0.25) (layer "F.Cu") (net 6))
 (segment (start 139.086791 106.445156) (end 139.518612 106.44159) (width 0.25) (layer "F.Cu") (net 6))
 (segment (start 135.24875 106.01751) (end 135.671924 106.04871) (width 0.25) (layer "F.Cu") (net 6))
 (segment (start 133.151352 106.271652) (end 130.3 107.2) (width 0.25) (layer "F.Cu") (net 6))
 (segment (start 136.515719 106.194411) (end 136.938282 106.268192) (width 0.25) (layer "F.Cu") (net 6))
 (segment (start 139.518612 106.44159) (end 142.81 106.315) (width 0.25) (layer "F.Cu") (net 6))
 (segment (start 137.362879 106.329185) (end 137.789124 106.377335) (width 0.25) (layer "F.Cu") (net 6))
 (segment (start 138.65506 106.435686) (end 139.086791 106.445156) (width 0.25) (layer "F.Cu") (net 6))
 (segment (start 133.562481 106.166659) (end 133.151352 106.271652) (width 0.25) (layer "F.Cu") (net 6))
 (segment (start 136.515719 106.194411) (end 136.092195 106.107215) (width 0.25) (layer "F.Cu") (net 6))
 (segment (start 130.3 107.2) (end 130.25 107.25) (width 0.25) (layer "B.Cu") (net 6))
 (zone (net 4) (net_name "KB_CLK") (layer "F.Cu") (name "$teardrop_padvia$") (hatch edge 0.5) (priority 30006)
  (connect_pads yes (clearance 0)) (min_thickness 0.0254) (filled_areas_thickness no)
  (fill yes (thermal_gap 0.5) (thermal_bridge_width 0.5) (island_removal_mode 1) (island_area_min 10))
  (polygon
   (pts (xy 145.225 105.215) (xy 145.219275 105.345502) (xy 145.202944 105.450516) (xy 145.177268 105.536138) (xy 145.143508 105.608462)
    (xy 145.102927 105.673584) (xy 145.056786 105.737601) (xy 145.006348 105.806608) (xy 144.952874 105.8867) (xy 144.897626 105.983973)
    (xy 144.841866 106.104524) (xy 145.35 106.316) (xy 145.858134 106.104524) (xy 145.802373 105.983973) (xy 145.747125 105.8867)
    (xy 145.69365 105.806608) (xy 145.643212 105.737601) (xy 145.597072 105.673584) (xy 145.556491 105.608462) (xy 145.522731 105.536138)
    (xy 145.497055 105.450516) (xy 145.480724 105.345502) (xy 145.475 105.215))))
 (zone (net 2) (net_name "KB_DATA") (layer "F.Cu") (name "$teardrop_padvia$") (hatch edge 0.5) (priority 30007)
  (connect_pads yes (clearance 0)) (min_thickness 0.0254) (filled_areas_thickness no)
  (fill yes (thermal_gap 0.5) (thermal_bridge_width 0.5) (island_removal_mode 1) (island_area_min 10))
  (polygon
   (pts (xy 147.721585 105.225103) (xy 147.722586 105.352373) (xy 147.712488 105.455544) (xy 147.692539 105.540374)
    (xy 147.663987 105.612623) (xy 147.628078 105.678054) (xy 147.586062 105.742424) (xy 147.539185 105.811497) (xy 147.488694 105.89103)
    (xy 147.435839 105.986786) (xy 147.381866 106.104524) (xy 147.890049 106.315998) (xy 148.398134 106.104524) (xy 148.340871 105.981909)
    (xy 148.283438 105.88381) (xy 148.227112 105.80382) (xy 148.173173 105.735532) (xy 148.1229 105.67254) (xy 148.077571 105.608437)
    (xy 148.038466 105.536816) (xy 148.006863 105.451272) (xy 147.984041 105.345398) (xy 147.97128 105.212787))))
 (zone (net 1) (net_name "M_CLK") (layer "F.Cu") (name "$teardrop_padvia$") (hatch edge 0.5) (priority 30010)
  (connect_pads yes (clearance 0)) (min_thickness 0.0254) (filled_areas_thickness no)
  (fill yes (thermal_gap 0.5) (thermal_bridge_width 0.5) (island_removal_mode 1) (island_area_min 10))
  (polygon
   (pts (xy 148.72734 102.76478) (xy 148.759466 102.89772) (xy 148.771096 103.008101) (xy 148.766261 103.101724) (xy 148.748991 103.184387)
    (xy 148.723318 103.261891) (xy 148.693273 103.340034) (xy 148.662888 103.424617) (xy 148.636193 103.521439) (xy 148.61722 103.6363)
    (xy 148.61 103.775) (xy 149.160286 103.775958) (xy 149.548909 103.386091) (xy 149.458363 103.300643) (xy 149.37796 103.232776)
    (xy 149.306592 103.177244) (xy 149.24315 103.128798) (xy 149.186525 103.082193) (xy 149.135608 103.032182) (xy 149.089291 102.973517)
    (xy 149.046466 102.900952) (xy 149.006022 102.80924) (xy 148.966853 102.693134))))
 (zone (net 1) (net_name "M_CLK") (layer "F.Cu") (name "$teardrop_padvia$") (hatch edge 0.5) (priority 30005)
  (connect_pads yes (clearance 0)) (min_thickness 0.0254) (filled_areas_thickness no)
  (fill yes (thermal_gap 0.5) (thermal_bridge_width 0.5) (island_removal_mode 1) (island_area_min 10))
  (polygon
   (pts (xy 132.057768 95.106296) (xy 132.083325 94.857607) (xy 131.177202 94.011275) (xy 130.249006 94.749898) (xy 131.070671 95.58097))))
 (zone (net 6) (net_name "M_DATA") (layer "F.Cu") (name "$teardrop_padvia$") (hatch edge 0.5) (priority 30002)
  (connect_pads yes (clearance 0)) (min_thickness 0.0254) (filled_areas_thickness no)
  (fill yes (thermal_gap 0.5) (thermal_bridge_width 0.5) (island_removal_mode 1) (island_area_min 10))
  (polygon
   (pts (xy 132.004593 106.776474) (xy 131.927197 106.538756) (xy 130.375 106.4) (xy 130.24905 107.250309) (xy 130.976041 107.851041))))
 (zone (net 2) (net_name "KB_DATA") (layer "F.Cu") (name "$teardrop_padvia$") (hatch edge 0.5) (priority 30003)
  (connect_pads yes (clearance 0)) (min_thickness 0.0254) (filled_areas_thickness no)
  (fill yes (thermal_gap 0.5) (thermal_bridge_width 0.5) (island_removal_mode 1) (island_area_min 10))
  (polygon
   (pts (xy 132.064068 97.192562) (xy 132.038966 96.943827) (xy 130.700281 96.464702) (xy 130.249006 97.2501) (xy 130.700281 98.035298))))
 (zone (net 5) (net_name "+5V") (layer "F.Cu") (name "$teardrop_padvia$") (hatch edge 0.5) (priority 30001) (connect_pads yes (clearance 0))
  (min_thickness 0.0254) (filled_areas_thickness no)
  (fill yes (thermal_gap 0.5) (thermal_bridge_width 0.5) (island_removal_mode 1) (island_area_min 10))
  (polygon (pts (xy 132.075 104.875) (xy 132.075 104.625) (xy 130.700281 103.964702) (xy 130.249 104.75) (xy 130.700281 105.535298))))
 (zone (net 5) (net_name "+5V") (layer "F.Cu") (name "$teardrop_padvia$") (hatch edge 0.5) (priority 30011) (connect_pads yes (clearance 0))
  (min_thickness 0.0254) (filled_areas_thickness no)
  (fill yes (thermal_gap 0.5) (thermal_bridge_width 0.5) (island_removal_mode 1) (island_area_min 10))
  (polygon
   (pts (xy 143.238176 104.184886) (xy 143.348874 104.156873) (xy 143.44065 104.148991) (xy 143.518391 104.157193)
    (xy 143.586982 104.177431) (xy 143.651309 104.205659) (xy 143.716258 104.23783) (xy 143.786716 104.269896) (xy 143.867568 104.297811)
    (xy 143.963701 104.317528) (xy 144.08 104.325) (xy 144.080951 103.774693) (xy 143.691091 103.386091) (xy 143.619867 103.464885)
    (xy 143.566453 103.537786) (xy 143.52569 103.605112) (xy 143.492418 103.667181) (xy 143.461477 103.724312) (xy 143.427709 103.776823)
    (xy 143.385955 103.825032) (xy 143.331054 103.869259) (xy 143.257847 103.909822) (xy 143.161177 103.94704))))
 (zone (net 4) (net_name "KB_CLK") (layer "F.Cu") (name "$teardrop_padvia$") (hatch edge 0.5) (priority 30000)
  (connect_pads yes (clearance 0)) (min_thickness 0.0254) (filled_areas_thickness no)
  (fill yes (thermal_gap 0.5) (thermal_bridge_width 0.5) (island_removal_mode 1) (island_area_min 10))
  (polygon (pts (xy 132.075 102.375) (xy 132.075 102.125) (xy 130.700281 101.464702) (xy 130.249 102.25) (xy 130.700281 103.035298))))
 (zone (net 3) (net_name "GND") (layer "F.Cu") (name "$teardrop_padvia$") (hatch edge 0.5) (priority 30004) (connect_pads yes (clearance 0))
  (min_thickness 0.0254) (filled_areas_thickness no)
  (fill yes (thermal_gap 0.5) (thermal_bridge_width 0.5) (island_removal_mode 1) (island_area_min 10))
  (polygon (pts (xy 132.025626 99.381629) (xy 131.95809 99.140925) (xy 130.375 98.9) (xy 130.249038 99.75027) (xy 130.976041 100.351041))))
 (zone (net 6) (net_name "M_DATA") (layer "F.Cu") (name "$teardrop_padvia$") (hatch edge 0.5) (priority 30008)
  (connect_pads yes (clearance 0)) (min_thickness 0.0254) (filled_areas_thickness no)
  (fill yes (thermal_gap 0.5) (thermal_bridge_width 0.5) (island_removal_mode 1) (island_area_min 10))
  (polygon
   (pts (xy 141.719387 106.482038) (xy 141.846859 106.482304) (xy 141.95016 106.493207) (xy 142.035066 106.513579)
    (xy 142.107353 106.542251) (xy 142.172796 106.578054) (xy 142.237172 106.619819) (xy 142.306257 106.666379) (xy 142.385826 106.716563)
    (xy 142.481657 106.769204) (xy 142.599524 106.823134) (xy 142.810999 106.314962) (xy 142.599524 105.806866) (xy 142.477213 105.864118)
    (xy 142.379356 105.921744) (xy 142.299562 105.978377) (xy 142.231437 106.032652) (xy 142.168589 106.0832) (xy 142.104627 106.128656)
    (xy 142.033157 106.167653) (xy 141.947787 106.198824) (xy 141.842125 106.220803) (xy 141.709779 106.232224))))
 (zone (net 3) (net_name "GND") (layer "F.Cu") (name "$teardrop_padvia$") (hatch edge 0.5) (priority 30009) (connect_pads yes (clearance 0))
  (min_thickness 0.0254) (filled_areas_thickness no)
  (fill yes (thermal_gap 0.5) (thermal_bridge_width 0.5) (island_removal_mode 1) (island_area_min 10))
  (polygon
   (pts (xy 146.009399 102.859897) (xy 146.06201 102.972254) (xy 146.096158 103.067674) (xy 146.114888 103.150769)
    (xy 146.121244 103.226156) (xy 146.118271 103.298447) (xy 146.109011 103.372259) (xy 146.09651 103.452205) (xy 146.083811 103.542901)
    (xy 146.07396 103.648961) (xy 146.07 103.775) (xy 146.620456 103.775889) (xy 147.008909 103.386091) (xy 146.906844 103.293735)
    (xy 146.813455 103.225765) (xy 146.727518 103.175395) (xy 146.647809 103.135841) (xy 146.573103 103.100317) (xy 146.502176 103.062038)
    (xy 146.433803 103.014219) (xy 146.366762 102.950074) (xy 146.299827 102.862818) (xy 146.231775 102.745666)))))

